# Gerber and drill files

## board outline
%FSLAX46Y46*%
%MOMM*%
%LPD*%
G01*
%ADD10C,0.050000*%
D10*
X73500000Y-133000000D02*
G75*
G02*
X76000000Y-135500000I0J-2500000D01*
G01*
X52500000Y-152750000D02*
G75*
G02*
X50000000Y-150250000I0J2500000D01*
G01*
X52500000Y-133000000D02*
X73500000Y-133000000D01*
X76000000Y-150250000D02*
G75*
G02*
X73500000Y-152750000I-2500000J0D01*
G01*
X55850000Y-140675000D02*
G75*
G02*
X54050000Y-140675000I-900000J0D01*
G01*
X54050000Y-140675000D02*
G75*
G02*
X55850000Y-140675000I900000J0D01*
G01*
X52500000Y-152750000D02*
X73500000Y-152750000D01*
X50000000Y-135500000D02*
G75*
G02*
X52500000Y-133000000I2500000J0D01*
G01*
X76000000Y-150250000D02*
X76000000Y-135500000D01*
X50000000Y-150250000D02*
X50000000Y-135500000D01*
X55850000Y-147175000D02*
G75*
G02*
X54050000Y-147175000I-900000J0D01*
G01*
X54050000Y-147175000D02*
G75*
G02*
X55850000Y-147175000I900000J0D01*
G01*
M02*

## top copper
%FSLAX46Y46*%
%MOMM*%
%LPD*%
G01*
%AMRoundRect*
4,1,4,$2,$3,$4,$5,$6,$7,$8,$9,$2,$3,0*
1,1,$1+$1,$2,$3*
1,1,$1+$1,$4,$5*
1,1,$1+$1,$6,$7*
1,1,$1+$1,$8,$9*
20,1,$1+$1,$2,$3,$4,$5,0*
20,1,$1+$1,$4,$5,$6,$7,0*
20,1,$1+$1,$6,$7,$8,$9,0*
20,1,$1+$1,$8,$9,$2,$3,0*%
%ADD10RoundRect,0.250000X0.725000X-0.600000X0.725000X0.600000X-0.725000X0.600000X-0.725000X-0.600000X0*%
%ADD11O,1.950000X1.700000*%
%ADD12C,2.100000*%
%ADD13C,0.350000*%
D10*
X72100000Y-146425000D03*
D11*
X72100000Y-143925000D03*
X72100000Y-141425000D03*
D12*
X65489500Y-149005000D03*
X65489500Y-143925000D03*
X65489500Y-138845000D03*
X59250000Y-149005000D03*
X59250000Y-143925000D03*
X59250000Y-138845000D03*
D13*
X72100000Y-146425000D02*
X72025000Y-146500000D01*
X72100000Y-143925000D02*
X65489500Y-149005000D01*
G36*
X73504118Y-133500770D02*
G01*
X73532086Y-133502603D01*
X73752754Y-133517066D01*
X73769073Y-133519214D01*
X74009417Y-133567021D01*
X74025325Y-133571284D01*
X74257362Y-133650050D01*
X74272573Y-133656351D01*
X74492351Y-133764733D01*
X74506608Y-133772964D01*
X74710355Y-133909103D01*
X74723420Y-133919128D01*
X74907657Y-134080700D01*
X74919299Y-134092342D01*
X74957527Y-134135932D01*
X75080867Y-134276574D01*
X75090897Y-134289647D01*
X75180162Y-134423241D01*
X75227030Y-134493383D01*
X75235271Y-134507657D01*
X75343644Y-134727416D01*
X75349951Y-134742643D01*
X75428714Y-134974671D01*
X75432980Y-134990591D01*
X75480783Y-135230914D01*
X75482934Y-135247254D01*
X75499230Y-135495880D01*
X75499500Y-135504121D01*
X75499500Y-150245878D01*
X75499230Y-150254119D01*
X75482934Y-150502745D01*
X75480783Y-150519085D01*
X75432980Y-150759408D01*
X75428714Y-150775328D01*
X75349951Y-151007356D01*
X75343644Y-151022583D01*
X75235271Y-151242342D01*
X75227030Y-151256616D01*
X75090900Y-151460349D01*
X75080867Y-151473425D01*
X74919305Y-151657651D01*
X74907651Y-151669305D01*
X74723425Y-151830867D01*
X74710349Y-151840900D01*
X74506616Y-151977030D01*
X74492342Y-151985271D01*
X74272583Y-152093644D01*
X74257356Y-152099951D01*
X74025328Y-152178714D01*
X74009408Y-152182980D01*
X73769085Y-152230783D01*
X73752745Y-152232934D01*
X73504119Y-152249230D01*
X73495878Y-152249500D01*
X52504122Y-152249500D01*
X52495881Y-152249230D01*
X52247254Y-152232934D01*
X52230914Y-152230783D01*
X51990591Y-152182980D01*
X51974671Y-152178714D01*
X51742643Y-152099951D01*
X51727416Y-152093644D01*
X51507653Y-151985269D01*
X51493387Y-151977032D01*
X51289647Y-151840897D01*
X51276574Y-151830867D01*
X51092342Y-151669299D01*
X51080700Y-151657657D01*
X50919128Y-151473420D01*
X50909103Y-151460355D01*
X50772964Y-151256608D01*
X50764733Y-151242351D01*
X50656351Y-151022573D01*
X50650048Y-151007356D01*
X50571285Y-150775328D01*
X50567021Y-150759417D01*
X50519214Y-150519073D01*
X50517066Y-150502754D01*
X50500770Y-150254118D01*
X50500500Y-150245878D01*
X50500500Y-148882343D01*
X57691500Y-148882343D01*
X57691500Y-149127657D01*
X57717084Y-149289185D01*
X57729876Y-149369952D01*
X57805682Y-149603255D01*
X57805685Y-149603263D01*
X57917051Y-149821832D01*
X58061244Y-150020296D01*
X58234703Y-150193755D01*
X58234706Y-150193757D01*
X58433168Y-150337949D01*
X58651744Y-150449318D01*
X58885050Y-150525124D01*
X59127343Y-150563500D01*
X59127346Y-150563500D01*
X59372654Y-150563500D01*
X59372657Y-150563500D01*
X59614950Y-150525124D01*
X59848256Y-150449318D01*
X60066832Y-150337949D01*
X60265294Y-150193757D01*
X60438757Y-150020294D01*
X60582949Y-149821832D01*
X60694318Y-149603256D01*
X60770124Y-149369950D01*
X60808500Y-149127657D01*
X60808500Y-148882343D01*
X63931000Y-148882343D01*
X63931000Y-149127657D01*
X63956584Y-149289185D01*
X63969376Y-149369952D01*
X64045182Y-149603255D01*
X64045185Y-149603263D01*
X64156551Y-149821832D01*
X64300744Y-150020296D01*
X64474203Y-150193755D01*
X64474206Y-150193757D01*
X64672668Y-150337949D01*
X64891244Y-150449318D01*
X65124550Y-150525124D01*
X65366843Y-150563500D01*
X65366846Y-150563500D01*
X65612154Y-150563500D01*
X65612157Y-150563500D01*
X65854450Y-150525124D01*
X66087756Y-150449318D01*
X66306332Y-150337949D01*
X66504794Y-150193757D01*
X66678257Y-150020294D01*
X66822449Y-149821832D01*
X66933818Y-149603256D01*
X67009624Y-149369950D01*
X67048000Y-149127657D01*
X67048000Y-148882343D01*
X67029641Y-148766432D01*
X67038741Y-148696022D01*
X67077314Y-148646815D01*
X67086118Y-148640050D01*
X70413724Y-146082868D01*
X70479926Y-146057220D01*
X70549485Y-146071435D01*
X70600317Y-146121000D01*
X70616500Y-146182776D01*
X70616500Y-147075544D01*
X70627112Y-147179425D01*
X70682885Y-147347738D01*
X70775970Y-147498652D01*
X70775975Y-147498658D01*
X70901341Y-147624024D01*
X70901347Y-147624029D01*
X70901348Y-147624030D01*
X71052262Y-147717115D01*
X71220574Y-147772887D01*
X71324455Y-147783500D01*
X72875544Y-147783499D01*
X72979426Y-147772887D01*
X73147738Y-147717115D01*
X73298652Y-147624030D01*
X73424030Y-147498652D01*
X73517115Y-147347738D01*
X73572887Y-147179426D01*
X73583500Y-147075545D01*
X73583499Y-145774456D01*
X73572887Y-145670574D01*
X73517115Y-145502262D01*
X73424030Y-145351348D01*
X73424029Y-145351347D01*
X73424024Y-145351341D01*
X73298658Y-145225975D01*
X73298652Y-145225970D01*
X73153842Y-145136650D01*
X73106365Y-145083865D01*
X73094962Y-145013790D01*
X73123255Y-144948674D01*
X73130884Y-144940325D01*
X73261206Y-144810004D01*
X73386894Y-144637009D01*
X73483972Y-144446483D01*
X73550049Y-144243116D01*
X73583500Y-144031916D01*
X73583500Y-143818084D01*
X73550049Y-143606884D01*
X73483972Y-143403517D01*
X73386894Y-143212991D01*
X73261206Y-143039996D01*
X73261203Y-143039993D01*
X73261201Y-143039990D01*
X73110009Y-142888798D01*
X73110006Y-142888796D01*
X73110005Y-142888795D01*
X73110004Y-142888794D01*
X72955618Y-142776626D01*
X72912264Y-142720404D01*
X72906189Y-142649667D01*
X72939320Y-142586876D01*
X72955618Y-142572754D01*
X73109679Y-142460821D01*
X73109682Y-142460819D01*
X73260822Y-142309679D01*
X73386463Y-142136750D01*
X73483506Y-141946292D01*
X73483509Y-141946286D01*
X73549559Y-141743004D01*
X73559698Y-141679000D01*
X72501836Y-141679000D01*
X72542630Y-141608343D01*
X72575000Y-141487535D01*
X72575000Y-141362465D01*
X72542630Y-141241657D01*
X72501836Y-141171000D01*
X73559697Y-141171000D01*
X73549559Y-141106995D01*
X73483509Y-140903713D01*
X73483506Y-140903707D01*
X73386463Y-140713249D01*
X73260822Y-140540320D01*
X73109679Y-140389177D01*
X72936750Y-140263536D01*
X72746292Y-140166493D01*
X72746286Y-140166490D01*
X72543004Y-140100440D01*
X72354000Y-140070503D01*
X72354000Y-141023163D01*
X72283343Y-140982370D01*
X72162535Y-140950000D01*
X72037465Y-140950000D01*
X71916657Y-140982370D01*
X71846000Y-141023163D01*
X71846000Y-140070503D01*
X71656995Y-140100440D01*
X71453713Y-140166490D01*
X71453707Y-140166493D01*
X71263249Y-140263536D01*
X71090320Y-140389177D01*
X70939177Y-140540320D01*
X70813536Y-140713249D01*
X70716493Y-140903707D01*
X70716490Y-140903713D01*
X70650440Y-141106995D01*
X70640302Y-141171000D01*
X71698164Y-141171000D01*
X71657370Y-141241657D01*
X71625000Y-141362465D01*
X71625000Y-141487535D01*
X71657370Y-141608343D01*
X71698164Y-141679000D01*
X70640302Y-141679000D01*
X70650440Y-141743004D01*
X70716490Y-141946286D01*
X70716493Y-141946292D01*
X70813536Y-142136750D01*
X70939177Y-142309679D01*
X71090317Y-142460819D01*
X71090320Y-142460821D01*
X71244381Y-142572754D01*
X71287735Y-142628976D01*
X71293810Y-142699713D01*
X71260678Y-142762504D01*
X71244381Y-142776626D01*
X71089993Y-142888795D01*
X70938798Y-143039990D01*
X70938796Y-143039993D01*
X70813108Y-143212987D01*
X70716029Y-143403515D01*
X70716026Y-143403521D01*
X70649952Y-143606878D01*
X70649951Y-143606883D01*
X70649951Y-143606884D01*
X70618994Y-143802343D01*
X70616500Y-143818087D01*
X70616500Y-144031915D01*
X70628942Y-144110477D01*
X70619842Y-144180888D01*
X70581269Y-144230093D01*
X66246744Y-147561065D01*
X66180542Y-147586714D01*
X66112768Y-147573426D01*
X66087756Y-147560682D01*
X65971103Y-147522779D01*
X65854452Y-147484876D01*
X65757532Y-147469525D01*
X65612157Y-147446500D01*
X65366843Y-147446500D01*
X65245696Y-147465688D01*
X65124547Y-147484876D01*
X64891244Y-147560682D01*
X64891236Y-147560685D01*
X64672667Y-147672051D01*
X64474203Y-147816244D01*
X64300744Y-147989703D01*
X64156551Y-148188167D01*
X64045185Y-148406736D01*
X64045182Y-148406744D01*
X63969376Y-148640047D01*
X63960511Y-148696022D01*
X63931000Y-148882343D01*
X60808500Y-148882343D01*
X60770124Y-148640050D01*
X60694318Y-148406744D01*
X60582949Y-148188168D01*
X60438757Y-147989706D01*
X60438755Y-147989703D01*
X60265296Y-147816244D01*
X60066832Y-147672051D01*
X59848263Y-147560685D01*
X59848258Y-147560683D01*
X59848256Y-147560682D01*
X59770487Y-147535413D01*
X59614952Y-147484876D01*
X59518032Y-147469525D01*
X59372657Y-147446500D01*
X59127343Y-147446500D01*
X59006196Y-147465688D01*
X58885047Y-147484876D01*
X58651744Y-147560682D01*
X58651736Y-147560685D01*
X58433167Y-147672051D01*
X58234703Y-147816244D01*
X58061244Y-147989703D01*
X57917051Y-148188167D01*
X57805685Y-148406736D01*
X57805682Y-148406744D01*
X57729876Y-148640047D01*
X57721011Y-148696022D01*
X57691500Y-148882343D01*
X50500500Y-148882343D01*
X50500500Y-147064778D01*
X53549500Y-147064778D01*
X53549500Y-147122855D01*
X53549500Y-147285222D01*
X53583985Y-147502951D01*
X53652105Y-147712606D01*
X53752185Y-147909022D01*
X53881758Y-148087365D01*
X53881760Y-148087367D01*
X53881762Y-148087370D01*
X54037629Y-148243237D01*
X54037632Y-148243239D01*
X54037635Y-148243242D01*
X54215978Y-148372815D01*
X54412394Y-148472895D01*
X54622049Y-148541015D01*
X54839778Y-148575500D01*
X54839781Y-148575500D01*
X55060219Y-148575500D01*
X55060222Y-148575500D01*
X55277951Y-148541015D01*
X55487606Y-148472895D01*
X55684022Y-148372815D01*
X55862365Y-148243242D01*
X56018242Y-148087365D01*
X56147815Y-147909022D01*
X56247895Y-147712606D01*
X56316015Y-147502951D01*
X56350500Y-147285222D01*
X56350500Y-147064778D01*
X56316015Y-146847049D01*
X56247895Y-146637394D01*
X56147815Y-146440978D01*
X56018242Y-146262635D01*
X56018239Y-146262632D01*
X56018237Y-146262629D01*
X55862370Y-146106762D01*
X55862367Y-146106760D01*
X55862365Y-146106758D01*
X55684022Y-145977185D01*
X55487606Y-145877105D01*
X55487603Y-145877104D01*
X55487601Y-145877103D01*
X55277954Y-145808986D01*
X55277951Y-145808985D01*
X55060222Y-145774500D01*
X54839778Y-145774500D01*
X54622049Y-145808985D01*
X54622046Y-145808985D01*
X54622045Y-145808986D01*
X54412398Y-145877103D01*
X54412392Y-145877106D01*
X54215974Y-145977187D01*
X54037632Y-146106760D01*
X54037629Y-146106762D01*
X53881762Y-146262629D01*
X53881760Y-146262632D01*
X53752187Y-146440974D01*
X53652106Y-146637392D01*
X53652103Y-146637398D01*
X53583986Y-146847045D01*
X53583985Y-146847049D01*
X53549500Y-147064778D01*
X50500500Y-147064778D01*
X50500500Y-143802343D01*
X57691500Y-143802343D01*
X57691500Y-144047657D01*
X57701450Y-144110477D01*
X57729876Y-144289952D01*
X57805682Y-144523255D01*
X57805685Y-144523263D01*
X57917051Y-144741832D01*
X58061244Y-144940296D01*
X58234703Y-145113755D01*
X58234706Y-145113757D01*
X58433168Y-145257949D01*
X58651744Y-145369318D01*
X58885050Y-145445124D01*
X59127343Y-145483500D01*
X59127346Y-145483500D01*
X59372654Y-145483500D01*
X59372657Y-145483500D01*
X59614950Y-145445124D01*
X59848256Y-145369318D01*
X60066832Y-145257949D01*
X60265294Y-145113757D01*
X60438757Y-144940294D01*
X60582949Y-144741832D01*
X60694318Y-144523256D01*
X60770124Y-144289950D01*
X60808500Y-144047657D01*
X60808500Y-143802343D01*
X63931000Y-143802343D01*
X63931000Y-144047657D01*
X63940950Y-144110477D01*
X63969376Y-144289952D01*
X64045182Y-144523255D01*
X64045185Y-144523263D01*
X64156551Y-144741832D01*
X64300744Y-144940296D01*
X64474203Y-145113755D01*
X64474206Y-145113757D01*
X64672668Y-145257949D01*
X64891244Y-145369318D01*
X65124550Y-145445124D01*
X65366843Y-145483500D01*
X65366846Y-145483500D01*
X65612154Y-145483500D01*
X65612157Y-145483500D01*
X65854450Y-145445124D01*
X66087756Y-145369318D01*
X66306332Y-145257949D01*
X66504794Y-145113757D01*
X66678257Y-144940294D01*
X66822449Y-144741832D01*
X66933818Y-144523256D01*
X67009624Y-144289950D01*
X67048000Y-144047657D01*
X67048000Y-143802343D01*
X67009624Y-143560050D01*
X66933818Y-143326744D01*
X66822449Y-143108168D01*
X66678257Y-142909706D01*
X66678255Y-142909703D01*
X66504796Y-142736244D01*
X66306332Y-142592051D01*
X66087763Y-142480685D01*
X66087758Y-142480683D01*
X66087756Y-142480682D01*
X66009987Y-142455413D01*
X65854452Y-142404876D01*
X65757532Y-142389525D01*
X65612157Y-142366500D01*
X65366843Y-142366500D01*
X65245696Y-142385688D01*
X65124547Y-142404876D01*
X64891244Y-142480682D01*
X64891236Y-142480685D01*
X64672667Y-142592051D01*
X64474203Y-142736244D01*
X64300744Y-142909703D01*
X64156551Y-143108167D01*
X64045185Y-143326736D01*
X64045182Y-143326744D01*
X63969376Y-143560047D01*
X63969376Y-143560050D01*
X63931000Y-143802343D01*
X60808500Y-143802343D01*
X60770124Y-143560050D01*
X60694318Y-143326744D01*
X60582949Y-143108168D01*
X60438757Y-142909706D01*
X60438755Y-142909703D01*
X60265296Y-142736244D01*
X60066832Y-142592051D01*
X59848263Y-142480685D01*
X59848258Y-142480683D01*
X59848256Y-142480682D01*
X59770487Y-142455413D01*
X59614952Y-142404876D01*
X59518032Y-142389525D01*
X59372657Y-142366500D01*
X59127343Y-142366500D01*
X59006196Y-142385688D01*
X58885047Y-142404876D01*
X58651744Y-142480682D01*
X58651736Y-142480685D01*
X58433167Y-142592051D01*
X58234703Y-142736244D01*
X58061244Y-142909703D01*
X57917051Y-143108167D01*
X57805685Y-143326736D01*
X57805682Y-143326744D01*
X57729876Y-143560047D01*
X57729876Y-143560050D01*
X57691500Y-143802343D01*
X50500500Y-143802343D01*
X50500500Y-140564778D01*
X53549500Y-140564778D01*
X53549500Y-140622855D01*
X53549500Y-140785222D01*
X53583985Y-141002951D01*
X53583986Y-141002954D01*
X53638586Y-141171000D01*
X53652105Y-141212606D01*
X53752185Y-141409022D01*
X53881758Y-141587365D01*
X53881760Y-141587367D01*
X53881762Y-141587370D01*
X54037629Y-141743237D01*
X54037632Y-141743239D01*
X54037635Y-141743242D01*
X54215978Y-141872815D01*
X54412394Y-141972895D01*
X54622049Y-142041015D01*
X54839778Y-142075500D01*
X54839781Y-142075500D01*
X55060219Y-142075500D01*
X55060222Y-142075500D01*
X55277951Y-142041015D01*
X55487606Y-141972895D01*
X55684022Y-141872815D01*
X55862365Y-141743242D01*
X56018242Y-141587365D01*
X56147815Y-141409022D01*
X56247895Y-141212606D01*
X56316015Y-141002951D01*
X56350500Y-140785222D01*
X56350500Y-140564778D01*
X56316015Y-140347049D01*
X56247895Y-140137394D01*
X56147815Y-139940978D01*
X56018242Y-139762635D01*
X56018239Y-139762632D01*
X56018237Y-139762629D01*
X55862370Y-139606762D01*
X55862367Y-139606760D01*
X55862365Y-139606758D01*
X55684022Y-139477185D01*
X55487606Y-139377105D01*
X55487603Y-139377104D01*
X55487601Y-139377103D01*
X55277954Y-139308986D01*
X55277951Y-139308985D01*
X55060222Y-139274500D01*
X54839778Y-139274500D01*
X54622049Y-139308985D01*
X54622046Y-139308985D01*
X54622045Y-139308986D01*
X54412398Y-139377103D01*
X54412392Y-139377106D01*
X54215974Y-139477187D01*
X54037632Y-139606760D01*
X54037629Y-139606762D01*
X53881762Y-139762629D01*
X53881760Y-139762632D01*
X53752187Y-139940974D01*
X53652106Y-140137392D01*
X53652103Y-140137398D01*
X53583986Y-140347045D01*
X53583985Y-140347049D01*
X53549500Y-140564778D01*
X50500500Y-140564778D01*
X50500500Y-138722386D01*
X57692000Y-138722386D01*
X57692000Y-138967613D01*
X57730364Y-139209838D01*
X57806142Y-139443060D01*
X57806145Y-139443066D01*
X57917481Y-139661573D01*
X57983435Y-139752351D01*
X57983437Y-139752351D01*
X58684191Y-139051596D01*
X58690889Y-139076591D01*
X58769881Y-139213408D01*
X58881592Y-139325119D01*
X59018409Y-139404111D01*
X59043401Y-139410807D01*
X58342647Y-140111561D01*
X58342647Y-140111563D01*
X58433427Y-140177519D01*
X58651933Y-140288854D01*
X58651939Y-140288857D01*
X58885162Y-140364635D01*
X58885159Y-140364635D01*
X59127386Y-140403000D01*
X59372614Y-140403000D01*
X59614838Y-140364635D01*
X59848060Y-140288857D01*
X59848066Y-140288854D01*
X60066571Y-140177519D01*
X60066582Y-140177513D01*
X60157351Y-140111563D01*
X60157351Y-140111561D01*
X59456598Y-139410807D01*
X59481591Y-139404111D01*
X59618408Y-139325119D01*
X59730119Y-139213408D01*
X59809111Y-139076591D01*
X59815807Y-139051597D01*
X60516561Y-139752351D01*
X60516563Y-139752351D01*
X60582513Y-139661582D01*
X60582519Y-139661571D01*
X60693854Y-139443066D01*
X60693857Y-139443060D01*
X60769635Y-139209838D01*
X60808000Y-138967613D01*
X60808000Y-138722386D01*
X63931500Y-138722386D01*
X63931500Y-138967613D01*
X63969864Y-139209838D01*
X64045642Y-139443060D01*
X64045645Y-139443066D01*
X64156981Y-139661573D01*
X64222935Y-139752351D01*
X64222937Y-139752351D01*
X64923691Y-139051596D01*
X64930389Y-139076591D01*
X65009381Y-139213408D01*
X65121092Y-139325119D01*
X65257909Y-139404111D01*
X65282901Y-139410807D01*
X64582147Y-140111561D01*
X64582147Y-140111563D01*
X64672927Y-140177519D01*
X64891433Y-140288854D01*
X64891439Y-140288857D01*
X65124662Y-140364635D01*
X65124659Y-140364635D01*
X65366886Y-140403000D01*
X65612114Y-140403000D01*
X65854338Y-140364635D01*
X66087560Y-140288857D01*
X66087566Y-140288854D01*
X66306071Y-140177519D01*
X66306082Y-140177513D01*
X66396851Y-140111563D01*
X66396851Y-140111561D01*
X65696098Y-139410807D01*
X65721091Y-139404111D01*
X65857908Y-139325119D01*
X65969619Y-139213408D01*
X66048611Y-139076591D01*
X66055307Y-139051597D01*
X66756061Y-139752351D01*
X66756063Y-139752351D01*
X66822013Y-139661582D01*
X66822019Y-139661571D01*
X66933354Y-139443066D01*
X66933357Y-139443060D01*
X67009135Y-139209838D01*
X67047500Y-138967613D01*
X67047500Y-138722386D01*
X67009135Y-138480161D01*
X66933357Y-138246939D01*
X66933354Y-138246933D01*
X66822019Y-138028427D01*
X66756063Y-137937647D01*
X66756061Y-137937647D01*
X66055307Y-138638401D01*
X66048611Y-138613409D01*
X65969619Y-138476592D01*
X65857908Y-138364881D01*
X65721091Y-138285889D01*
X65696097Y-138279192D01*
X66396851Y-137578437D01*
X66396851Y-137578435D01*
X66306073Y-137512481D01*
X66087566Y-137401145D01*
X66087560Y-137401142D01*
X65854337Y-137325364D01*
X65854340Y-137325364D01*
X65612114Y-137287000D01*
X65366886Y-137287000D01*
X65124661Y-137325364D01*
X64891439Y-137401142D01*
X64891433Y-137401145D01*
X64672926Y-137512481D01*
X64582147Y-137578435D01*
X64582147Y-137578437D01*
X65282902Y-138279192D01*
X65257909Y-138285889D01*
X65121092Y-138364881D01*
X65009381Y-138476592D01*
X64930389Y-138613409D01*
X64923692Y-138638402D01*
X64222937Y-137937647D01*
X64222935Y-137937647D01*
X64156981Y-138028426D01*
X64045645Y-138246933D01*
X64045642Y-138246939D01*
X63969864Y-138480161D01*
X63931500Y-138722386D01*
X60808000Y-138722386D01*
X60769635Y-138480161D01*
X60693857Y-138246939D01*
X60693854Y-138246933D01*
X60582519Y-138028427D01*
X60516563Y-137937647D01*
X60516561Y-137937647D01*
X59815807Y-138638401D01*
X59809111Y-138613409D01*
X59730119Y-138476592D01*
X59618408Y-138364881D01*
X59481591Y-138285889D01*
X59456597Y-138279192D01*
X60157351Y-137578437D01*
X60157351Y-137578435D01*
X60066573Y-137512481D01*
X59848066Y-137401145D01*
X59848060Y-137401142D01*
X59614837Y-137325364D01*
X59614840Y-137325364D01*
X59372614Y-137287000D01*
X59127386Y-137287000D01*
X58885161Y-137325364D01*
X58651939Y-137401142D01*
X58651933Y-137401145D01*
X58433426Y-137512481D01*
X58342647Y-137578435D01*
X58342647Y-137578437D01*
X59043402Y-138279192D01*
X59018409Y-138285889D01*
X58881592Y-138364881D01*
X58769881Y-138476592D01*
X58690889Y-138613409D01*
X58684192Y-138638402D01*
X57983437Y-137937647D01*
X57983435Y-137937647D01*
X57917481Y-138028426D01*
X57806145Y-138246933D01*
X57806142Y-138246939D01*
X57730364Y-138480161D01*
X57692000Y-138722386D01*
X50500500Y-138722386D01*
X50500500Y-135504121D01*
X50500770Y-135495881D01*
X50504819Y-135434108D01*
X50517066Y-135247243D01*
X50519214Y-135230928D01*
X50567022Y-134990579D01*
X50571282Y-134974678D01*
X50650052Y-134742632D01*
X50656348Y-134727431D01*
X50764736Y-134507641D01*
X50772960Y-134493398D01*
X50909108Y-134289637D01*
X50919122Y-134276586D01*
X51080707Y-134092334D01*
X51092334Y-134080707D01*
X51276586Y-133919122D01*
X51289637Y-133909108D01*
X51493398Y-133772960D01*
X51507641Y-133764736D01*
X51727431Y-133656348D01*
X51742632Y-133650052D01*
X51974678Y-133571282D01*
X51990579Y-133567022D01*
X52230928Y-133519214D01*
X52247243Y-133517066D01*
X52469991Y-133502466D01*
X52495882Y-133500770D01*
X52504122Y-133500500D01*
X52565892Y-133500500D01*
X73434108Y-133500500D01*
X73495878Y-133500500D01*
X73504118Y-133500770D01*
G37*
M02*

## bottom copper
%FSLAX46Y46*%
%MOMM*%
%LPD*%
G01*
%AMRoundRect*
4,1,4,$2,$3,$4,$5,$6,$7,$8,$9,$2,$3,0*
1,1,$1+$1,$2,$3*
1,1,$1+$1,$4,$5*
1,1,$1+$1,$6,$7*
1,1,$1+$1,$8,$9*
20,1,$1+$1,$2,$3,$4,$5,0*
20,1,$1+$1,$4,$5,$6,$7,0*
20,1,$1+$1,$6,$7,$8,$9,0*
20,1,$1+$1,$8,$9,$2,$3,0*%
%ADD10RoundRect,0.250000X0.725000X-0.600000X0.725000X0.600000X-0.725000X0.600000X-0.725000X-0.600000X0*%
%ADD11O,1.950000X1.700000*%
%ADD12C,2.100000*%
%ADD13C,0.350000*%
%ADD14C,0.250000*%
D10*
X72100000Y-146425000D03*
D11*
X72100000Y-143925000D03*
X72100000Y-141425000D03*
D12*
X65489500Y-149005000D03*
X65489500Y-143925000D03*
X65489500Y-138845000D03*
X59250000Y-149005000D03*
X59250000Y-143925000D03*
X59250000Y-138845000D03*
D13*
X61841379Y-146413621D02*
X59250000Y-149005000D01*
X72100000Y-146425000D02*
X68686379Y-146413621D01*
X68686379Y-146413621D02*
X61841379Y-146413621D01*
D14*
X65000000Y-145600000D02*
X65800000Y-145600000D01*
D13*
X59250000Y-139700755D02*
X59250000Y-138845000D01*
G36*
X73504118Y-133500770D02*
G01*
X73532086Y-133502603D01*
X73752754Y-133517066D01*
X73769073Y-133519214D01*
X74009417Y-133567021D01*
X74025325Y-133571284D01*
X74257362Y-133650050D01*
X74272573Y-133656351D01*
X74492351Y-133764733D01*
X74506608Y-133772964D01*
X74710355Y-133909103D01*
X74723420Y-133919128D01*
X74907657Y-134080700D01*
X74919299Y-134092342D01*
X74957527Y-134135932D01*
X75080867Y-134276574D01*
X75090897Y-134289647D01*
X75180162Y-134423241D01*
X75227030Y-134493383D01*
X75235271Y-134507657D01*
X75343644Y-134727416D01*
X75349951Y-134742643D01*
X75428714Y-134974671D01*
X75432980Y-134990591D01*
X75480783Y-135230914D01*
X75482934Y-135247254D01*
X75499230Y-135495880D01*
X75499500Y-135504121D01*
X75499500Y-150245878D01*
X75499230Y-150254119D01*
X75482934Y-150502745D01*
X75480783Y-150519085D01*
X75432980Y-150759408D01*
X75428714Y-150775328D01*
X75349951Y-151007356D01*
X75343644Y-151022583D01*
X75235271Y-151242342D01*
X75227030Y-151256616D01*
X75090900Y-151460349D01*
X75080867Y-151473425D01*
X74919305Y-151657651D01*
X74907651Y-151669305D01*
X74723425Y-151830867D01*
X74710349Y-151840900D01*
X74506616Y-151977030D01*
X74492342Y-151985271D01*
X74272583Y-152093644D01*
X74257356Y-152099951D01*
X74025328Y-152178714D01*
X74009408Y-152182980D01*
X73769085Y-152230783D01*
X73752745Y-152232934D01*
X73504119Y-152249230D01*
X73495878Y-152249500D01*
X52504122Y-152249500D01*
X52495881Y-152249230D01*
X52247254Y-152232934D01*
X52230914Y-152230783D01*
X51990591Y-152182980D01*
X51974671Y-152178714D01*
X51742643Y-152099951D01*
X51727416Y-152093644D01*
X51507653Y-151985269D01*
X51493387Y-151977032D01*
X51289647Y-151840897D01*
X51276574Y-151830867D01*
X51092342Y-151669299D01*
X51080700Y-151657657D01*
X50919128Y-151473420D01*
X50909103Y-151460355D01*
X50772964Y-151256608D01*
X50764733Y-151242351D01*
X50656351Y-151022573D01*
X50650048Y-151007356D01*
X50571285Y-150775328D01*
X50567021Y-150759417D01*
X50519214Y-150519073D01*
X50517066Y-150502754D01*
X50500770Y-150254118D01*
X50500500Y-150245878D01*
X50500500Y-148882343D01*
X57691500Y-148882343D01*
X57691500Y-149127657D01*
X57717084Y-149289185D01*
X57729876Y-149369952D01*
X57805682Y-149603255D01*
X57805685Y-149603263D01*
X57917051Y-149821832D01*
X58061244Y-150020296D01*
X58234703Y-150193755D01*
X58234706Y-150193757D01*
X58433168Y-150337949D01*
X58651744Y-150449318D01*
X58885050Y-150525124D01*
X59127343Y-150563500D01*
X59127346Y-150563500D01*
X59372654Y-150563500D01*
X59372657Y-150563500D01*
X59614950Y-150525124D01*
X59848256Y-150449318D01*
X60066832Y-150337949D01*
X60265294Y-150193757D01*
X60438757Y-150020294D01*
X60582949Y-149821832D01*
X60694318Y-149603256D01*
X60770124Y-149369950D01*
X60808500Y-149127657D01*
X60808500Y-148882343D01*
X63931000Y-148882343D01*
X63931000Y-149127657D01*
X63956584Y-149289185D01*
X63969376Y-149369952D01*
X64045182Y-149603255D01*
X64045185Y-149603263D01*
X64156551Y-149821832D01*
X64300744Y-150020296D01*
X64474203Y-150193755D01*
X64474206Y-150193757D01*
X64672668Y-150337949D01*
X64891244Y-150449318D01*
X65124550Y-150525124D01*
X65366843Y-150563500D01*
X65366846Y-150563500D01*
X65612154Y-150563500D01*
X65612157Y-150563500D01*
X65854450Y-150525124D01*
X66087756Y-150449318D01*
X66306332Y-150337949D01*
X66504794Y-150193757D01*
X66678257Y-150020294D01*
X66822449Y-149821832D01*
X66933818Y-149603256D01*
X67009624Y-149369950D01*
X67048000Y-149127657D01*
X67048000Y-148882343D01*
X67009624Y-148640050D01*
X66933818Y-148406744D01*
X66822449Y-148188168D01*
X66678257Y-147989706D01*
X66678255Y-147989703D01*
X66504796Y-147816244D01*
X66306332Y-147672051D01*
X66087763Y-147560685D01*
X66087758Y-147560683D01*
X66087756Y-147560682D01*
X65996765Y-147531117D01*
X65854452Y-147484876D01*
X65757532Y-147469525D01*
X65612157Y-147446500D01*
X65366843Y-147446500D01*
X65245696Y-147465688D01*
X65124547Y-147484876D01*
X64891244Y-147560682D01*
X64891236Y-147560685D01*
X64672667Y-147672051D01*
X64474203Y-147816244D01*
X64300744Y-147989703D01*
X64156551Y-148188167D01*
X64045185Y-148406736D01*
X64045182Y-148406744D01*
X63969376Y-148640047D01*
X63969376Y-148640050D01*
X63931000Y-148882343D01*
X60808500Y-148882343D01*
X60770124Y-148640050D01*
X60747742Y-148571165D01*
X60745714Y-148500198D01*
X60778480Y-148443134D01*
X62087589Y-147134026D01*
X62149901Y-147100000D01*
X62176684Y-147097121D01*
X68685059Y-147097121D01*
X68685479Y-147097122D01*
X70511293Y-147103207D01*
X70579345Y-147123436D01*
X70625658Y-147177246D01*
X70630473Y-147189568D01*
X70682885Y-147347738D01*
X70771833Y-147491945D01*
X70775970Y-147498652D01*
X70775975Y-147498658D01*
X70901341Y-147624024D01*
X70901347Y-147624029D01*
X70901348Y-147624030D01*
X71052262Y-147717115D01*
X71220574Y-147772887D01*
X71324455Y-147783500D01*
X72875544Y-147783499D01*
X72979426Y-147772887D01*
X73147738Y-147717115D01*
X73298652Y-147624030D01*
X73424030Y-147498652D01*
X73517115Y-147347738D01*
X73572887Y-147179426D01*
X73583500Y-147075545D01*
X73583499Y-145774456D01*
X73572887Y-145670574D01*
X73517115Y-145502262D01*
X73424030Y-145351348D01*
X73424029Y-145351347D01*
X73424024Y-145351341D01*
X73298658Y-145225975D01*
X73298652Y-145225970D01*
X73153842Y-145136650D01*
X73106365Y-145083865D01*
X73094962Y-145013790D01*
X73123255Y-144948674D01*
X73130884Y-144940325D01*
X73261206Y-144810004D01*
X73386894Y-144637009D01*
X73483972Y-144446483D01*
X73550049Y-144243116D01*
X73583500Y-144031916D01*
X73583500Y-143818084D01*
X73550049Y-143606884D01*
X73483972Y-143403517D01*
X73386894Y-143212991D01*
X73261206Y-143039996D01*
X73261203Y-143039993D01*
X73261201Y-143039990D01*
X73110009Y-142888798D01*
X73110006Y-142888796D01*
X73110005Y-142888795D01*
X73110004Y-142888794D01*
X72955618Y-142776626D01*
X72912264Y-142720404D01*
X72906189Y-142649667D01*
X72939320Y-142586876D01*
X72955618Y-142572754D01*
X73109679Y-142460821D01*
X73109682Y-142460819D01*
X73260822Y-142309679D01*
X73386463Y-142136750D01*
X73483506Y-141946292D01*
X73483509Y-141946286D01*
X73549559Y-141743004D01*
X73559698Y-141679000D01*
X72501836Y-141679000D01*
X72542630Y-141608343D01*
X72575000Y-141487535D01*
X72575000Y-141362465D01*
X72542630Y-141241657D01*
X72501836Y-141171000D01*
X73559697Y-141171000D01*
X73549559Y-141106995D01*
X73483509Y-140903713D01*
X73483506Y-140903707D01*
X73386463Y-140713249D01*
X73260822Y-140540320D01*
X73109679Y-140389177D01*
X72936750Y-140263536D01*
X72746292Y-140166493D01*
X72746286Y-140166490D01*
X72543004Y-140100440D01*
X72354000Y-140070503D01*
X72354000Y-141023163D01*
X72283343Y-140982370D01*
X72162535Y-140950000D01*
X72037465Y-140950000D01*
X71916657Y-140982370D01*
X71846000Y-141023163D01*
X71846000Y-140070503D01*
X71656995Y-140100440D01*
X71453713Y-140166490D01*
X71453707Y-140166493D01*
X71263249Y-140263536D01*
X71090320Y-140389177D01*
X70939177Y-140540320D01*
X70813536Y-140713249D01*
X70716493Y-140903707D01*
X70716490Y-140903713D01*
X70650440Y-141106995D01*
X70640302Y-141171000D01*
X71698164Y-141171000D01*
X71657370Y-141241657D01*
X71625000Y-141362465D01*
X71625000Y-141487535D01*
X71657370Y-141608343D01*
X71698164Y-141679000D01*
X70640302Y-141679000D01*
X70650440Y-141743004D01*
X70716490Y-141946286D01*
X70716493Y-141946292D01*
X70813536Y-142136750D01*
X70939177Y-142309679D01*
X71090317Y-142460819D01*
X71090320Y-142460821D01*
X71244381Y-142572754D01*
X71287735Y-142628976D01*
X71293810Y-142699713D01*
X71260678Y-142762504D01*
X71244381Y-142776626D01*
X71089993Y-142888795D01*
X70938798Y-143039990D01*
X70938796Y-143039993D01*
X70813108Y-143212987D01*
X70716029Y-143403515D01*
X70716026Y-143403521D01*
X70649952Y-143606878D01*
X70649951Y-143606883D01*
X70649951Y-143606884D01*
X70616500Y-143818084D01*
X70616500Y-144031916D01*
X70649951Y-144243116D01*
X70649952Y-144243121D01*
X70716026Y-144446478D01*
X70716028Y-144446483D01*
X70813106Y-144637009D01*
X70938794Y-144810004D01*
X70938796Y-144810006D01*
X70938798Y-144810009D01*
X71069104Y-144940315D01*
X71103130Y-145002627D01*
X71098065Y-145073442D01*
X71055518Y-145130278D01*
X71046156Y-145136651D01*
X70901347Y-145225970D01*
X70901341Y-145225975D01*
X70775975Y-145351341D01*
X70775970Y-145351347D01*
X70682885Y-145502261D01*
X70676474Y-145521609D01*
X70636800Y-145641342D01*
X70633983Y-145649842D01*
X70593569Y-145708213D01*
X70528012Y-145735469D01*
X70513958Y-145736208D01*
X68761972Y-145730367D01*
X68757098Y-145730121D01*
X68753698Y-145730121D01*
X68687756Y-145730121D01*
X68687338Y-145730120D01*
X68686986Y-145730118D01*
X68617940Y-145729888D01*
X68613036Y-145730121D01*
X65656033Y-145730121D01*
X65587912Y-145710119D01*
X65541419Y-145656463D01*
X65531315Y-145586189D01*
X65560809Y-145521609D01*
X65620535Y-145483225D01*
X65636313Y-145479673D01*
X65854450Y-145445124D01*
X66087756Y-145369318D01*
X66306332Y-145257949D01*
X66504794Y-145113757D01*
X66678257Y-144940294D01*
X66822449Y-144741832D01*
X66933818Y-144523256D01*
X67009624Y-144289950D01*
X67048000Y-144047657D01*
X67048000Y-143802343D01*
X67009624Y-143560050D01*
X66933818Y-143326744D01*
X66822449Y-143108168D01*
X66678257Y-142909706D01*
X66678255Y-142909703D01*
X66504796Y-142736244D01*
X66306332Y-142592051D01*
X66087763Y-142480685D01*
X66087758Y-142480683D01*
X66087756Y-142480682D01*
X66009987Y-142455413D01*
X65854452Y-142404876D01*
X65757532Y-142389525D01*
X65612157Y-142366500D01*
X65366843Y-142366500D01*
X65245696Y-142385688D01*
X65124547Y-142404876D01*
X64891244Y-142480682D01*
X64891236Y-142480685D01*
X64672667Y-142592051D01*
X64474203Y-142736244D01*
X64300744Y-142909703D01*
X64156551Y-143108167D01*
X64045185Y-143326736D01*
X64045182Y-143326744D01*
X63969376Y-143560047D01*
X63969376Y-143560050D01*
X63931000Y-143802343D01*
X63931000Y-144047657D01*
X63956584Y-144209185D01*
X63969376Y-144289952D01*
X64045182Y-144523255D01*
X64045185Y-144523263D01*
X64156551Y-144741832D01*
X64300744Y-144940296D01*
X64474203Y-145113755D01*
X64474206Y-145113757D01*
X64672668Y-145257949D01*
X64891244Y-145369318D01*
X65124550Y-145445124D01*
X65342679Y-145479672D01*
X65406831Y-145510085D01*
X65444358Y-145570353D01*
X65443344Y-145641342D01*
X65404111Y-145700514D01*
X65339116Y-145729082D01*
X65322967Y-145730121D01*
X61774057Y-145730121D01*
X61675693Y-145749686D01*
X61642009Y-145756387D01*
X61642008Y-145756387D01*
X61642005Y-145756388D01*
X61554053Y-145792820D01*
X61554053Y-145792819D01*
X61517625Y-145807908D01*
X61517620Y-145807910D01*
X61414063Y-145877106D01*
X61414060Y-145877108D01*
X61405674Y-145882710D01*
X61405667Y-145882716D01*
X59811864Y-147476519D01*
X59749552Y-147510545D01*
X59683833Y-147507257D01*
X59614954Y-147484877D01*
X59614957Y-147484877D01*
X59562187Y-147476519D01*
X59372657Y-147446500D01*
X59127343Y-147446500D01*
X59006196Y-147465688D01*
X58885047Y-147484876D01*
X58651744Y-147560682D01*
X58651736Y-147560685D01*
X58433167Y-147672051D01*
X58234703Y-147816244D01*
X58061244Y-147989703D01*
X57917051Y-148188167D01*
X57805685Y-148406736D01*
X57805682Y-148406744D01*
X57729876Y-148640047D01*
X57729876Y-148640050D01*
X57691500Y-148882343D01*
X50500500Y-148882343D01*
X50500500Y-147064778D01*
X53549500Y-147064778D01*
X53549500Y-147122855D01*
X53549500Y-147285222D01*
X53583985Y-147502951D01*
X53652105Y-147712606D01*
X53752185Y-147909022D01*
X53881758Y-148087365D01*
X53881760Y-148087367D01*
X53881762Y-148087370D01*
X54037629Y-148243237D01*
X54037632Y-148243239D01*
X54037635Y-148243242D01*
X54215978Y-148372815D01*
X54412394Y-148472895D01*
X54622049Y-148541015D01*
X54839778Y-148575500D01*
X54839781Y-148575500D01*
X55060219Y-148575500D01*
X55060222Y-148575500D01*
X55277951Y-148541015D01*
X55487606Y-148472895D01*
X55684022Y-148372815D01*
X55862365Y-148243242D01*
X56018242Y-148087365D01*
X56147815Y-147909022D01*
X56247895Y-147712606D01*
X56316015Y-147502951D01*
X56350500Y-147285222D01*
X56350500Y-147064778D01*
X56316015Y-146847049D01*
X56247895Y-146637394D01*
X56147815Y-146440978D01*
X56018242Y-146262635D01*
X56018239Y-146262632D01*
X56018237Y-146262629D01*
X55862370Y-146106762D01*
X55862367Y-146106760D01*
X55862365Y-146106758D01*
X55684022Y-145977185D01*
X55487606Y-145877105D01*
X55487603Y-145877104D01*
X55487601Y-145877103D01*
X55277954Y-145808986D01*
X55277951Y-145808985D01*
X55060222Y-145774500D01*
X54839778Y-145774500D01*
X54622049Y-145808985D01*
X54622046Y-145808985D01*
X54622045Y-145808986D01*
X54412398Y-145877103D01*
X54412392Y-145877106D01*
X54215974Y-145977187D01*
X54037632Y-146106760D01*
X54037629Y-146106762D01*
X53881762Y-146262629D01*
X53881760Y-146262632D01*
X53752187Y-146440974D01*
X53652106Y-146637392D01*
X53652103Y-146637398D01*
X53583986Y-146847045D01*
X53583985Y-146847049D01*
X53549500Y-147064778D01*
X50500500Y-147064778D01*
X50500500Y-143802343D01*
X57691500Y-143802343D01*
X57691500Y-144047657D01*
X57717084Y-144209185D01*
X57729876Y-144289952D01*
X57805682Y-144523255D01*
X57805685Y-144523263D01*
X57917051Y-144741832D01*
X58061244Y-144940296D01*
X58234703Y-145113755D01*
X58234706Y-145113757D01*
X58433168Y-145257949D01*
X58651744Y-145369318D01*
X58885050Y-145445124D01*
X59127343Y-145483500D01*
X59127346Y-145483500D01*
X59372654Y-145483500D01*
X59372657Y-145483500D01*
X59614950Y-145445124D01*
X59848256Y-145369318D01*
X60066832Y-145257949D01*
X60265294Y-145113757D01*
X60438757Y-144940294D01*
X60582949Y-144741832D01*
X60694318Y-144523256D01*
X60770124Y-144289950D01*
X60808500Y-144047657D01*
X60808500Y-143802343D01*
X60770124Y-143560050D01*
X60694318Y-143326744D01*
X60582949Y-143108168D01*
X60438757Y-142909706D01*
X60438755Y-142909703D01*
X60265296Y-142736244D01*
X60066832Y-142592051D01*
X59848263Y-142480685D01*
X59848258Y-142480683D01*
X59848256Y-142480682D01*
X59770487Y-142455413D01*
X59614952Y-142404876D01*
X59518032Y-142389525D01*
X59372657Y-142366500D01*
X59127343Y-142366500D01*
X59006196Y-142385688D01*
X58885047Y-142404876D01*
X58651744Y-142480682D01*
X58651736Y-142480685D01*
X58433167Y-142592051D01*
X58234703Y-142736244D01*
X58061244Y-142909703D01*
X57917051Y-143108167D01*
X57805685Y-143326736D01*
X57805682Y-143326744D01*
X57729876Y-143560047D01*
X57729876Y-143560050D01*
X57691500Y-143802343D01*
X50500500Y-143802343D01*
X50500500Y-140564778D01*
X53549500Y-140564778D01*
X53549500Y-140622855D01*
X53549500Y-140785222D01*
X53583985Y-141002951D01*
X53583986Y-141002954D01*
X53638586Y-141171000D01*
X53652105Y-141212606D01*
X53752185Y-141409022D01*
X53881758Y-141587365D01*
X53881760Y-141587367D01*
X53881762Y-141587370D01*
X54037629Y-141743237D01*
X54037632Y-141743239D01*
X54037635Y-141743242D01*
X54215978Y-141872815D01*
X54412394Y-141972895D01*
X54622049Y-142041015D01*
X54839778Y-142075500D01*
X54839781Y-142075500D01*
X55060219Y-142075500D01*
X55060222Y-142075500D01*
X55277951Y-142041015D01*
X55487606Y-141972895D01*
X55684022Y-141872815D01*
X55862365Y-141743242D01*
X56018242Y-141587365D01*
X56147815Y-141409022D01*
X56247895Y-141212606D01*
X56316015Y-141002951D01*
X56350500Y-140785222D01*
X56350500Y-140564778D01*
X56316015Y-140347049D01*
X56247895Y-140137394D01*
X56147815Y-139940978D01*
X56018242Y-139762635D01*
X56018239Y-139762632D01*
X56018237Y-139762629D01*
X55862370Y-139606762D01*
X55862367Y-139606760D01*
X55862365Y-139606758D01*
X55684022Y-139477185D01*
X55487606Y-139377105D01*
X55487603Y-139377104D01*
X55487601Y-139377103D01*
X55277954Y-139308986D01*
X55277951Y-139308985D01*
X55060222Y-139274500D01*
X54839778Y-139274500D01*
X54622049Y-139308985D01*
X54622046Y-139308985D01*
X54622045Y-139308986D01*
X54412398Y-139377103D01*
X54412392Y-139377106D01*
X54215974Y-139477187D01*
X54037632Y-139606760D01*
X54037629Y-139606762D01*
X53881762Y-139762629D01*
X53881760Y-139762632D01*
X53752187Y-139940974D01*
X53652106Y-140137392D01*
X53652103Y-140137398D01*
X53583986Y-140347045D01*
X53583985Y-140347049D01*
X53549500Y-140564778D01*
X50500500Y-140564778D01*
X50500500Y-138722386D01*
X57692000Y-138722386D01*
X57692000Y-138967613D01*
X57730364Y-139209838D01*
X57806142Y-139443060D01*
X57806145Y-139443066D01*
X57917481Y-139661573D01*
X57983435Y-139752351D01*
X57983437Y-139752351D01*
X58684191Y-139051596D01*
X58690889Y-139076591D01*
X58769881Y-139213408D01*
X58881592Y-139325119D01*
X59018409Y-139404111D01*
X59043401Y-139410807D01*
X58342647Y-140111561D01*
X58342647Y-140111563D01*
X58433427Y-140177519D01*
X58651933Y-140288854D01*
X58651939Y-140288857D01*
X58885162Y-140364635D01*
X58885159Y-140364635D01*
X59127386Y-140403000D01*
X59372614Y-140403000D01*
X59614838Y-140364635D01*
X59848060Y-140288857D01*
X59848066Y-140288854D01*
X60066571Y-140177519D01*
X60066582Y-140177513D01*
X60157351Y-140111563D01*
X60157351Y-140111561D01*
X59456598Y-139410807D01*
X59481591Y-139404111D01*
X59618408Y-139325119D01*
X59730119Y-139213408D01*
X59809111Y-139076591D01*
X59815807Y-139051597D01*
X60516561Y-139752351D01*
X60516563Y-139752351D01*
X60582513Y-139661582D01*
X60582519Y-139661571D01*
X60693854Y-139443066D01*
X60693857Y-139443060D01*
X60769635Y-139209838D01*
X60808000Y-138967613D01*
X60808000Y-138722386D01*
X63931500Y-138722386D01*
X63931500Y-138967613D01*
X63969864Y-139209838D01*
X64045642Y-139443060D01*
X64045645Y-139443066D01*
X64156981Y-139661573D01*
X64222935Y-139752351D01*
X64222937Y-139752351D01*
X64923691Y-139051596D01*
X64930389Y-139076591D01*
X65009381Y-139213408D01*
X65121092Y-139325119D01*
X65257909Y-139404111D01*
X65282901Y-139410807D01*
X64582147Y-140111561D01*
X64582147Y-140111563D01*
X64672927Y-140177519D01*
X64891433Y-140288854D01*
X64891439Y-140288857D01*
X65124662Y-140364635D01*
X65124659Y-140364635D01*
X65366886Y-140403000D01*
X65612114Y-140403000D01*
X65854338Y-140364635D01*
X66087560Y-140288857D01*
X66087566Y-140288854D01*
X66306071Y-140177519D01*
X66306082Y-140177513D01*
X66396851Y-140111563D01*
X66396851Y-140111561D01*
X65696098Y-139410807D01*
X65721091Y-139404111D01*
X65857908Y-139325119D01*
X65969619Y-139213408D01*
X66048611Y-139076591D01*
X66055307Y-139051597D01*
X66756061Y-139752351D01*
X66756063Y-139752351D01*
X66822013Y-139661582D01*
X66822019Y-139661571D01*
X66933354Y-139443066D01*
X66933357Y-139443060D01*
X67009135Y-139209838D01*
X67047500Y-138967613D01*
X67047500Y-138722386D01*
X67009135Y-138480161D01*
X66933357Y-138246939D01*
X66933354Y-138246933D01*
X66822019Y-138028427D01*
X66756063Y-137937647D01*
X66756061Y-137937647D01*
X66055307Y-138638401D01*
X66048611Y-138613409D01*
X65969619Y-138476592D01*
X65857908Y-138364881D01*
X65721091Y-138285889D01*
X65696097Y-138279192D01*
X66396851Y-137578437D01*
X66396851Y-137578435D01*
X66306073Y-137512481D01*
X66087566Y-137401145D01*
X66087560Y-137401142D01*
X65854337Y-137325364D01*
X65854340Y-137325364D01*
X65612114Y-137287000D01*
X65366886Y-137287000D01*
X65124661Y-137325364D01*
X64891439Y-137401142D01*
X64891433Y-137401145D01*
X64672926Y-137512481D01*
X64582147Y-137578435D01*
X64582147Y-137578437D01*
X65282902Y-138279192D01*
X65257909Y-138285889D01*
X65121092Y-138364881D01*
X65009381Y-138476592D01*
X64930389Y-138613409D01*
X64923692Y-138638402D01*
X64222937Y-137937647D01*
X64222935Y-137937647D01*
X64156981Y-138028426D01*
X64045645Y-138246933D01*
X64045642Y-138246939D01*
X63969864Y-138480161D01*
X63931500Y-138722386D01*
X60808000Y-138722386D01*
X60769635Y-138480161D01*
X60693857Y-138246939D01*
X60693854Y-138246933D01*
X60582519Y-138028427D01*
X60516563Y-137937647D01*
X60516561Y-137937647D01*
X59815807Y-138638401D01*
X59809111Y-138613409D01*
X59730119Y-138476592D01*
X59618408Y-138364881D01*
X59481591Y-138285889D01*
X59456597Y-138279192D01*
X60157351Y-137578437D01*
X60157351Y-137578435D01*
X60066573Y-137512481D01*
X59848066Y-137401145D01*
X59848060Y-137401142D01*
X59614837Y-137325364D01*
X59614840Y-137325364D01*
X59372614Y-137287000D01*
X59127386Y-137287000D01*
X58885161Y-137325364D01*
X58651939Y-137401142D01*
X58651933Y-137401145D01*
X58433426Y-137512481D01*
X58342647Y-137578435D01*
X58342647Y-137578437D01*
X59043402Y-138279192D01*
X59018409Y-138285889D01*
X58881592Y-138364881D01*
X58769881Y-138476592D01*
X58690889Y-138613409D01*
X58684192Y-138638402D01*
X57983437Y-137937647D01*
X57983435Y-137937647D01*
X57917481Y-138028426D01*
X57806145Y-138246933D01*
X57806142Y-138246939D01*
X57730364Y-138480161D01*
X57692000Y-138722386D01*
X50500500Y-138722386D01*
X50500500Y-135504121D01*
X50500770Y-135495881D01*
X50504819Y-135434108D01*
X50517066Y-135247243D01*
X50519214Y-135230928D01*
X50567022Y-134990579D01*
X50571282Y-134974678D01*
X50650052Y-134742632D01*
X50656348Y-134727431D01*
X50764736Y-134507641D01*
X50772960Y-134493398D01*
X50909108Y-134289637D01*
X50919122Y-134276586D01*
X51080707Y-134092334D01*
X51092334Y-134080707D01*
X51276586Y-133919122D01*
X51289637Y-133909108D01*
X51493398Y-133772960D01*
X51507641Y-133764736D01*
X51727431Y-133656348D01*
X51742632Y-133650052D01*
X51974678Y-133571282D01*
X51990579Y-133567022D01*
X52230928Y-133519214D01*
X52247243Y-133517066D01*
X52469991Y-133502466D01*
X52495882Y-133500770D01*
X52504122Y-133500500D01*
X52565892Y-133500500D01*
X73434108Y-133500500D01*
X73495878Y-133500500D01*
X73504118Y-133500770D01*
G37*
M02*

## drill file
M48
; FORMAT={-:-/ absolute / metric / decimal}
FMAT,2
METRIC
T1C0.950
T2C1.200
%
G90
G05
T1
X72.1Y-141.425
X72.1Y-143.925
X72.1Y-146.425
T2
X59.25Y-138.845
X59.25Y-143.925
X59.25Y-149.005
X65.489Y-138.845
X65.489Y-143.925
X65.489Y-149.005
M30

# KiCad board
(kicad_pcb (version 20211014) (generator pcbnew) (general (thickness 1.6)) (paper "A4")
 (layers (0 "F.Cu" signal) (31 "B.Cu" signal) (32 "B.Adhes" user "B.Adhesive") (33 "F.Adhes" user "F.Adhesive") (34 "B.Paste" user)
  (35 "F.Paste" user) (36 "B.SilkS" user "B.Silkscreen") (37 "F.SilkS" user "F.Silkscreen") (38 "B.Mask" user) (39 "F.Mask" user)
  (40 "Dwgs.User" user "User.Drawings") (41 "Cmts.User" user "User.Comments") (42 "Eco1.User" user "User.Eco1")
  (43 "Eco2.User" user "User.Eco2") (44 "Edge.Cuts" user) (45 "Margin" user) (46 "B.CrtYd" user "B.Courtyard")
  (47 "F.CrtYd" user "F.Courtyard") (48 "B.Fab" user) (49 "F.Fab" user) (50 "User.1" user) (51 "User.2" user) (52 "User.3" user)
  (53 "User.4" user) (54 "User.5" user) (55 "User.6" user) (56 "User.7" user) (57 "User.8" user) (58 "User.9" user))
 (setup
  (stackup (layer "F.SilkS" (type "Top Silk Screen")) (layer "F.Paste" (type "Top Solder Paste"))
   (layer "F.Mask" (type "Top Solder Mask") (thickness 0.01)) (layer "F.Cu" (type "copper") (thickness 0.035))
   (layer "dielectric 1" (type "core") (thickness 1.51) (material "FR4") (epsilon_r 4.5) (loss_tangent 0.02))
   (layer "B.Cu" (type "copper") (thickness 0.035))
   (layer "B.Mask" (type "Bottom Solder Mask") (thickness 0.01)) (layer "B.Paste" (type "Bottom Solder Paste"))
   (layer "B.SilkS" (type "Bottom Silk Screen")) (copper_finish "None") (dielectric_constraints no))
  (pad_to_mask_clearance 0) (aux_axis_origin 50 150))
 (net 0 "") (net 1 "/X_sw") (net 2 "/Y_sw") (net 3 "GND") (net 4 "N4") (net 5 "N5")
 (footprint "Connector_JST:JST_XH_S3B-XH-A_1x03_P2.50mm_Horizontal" (layer "F.Cu") (at 72.1 146.425 90)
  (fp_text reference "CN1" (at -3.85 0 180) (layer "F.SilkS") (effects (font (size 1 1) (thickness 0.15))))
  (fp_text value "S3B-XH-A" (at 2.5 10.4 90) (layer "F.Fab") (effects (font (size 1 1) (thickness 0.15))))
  (pad "1" thru_hole roundrect (at 0 0 90) (size 1.7 1.95) (drill 0.95) (layers *.Cu *.Mask) (roundrect_rratio 0.1470588235) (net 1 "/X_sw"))
  (pad "2" thru_hole oval (at 2.5 0 90) (size 1.7 1.95) (drill 0.95) (layers *.Cu *.Mask) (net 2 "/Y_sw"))
  (pad "3" thru_hole oval (at 5 0 90) (size 1.7 1.95) (drill 0.95) (layers *.Cu *.Mask) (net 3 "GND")))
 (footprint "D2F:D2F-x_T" (layer "F.Cu") (at 65.4895 149.005 90)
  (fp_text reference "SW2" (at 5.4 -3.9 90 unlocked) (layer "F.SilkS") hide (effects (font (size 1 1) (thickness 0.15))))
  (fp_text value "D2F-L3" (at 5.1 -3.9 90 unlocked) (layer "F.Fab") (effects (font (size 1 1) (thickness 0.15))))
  (pad "1" thru_hole circle (at 0 0 90) (size 2.1 2.1) (drill 1.2) (layers *.Cu *.Mask) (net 2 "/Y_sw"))
  (pad "2" thru_hole circle (at 5.08 0 90) (size 2.1 2.1) (drill 1.2) (layers *.Cu *.Mask) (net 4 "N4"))
  (pad "3" thru_hole circle (at 10.16 0 90) (size 2.1 2.1) (drill 1.2) (layers *.Cu *.Mask) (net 3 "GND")))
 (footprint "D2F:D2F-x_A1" (layer "B.Cu") (at 52.75 147.175 90)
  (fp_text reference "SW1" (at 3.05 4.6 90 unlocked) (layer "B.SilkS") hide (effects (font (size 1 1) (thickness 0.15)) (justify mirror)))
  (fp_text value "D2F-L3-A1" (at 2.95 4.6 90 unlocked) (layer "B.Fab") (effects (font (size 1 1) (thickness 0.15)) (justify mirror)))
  (pad "1" thru_hole circle (at -1.83 6.5 90) (size 2.1 2.1) (drill 1.2) (layers *.Cu *.Mask) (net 1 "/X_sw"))
  (pad "2" thru_hole circle (at 3.25 6.5 90) (size 2.1 2.1) (drill 1.2) (layers *.Cu *.Mask) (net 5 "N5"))
  (pad "3" thru_hole circle (at 8.33 6.5 90) (size 2.1 2.1) (drill 1.2) (layers *.Cu *.Mask) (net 3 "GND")))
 (gr_arc (start 73.5 133) (mid 75.267767 133.732233) (end 76 135.5) (layer "Edge.Cuts") (width 0.05))
 (gr_arc (start 52.5 152.75) (mid 50.732233 152.017767) (end 50 150.25) (layer "Edge.Cuts") (width 0.05))
 (gr_line (start 52.5 133) (end 73.5 133) (layer "Edge.Cuts") (width 0.05))
 (gr_arc (start 76 150.25) (mid 75.267767 152.017767) (end 73.5 152.75) (layer "Edge.Cuts") (width 0.05))
 (gr_circle (center 54.95 140.675) (end 55.85 140.675) (layer "Edge.Cuts") (width 0.05) (fill none))
 (gr_line (start 52.5 152.75) (end 73.5 152.75) (layer "Edge.Cuts") (width 0.05))
 (gr_arc (start 50 135.5) (mid 50.732233 133.732233) (end 52.5 133) (layer "Edge.Cuts") (width 0.05))
 (gr_line (start 76 150.25) (end 76 135.5) (layer "Edge.Cuts") (width 0.05))
 (gr_line (start 50 150.25) (end 50 135.5) (layer "Edge.Cuts") (width 0.05))
 (gr_circle (center 54.95 147.175) (end 55.85 147.175) (layer "Edge.Cuts") (width 0.05) (fill none))
 (segment (start 72.1 146.425) (end 72.025 146.5) (width 0.35) (layer "F.Cu") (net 1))
 (segment (start 61.841379 146.413621) (end 59.25 149.005) (width 0.35) (layer "B.Cu") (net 1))
 (segment (start 72.1 146.425) (end 68.686379 146.413621) (width 0.35) (layer "B.Cu") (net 1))
 (segment (start 68.686379 146.413621) (end 61.841379 146.413621) (width 0.35) (layer "B.Cu") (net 1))
 (segment (start 72.1 143.925) (end 65.4895 149.005) (width 0.35) (layer "F.Cu") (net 2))
 (segment (start 65 145.6) (end 65.8 145.6) (width 0.25) (layer "B.Cu") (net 3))
 (segment (start 59.25 139.700755) (end 59.25 138.845) (width 0.35) (layer "B.Cu") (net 3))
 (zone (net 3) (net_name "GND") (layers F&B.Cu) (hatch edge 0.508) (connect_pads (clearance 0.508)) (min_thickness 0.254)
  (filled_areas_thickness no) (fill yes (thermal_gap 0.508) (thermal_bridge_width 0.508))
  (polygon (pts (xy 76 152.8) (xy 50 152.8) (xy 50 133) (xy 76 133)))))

